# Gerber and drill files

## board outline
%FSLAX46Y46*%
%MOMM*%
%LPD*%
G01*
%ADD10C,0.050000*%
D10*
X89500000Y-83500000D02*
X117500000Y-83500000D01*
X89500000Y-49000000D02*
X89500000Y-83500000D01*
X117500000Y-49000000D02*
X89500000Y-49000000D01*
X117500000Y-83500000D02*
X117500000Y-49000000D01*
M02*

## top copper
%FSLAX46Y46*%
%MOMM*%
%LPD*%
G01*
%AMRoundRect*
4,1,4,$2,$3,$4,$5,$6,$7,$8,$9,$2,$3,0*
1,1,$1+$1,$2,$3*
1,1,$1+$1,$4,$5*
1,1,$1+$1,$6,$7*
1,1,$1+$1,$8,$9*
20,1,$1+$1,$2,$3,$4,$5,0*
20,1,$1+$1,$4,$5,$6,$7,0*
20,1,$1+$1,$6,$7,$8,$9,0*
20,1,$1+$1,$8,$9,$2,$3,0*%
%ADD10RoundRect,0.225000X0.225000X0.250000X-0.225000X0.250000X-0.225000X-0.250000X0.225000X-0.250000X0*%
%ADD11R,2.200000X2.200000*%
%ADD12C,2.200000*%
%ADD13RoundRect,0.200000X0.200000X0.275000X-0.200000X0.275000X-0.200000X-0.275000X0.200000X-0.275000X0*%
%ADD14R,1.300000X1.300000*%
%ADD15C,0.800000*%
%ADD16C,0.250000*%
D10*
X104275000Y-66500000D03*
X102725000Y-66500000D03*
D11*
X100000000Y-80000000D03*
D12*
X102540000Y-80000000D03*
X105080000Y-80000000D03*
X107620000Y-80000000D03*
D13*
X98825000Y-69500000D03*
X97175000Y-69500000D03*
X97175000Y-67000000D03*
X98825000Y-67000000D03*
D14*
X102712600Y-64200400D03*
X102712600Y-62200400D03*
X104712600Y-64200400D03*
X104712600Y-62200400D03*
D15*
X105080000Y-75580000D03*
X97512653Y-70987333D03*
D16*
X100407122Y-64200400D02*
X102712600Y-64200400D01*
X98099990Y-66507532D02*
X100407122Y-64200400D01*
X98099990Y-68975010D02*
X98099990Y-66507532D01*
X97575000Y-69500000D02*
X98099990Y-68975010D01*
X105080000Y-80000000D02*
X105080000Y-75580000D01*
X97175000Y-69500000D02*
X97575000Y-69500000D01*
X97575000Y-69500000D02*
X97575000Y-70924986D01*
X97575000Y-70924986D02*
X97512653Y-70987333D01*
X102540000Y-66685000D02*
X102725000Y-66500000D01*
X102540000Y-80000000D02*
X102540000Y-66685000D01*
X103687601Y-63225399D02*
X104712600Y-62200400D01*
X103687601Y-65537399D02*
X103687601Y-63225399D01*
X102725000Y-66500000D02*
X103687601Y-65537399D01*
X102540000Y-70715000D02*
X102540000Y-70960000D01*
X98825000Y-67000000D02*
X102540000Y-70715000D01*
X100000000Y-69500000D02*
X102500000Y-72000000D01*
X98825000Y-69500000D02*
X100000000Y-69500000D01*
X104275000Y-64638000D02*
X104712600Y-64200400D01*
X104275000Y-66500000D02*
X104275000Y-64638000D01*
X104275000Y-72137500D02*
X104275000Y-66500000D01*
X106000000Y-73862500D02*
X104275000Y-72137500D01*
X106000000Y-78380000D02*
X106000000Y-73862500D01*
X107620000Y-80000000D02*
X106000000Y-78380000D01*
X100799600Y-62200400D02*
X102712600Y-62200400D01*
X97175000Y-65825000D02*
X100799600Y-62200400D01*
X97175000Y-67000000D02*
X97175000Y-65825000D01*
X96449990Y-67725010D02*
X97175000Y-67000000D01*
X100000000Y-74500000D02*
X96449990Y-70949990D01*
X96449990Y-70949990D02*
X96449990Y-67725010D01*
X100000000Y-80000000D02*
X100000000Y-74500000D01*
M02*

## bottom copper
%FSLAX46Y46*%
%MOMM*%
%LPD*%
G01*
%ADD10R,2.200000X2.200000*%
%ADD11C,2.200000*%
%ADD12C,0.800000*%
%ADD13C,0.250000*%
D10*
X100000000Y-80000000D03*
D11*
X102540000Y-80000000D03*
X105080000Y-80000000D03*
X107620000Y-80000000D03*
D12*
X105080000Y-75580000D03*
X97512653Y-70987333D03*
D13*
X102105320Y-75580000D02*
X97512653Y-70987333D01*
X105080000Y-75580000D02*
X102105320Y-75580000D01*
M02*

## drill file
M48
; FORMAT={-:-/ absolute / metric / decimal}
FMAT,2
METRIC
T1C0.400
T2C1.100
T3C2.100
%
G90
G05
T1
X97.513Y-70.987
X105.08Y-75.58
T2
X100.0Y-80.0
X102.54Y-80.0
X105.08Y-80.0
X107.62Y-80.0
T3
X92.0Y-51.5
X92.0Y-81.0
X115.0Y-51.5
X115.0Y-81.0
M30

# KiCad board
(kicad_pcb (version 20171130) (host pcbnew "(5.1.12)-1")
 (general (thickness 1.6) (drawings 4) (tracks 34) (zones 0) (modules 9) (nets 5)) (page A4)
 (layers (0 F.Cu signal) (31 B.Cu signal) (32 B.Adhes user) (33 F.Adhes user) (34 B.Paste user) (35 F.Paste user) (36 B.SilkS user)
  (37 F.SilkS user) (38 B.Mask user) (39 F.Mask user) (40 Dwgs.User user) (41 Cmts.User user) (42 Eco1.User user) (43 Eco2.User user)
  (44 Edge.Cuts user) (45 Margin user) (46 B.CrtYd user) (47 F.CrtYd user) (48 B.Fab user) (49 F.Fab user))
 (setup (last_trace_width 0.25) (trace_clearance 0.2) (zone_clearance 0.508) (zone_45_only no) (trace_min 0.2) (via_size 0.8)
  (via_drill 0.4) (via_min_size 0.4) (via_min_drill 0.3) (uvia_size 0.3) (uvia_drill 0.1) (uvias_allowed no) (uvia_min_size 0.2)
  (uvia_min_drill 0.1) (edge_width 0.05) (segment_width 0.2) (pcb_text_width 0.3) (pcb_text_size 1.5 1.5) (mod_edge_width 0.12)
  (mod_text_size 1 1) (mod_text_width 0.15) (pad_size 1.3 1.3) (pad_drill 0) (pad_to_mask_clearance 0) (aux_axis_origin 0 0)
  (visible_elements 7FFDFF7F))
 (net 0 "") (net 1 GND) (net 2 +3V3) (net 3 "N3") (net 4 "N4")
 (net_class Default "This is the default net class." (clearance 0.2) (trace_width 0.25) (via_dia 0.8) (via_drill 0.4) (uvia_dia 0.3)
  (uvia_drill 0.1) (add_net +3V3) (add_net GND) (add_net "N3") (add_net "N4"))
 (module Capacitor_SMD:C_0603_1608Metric (layer F.Cu) (at 103.5 66.5 180)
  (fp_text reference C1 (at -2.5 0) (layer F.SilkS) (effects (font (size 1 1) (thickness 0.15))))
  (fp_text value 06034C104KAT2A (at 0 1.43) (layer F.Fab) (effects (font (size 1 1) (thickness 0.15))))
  (pad 1 smd roundrect (at -0.775 0 180) (size 0.9 0.95) (layers F.Cu F.Paste F.Mask) (roundrect_rratio 0.25) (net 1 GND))
  (pad 2 smd roundrect (at 0.775 0 180) (size 0.9 0.95) (layers F.Cu F.Paste F.Mask) (roundrect_rratio 0.25) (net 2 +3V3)))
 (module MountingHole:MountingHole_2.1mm (layer F.Cu) (at 92 81)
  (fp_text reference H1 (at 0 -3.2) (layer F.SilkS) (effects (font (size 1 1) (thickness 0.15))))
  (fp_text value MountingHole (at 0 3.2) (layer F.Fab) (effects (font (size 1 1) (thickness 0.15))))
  (pad "" np_thru_hole circle (at 0 0) (size 2.1 2.1) (drill 2.1) (layers *.Cu *.Mask)))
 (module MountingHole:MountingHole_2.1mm (layer F.Cu) (at 92 51.5)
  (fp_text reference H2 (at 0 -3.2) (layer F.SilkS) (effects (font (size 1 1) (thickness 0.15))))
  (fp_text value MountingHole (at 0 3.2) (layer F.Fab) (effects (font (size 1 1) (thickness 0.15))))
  (pad "" np_thru_hole circle (at 0 0) (size 2.1 2.1) (drill 2.1) (layers *.Cu *.Mask)))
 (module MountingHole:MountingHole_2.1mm (layer F.Cu) (at 115 51.5)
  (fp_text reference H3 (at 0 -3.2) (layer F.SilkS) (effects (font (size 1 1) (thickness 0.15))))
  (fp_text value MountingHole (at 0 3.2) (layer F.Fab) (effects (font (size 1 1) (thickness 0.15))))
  (pad "" np_thru_hole circle (at 0 0) (size 2.1 2.1) (drill 2.1) (layers *.Cu *.Mask)))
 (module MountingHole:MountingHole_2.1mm (layer F.Cu) (at 115 81)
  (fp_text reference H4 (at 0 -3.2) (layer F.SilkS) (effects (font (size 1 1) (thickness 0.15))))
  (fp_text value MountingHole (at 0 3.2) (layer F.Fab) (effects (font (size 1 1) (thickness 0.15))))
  (pad "" np_thru_hole circle (at 0 0) (size 2.1 2.1) (drill 2.1) (layers *.Cu *.Mask)))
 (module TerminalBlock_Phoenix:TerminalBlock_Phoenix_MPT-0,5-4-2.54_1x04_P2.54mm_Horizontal (layer F.Cu) (at 100 80)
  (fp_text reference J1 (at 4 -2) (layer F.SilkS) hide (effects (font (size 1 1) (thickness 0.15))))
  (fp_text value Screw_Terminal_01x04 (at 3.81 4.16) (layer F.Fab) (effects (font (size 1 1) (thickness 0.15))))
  (pad 1 thru_hole rect (at 0 0) (size 2.2 2.2) (drill 1.1) (layers *.Cu *.Mask) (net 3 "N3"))
  (pad 2 thru_hole circle (at 2.54 0) (size 2.2 2.2) (drill 1.1) (layers *.Cu *.Mask) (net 2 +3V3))
  (pad 3 thru_hole circle (at 5.08 0) (size 2.2 2.2) (drill 1.1) (layers *.Cu *.Mask) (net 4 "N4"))
  (pad 4 thru_hole circle (at 7.62 0) (size 2.2 2.2) (drill 1.1) (layers *.Cu *.Mask) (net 1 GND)))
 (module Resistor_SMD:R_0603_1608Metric (layer F.Cu) (at 98 69.5 180)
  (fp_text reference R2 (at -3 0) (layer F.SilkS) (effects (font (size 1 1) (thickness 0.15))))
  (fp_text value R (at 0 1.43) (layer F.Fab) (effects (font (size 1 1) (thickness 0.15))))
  (pad 1 smd roundrect (at -0.825 0 180) (size 0.8 0.95) (layers F.Cu F.Paste F.Mask) (roundrect_rratio 0.25) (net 2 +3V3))
  (pad 2 smd roundrect (at 0.825 0 180) (size 0.8 0.95) (layers F.Cu F.Paste F.Mask) (roundrect_rratio 0.25) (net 4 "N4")))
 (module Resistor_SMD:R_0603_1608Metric (layer F.Cu) (at 98 67 180)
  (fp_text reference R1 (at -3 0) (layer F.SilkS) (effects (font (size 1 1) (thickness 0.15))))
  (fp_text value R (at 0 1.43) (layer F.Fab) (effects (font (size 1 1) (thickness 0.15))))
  (pad 2 smd roundrect (at 0.825 0 180) (size 0.8 0.95) (layers F.Cu F.Paste F.Mask) (roundrect_rratio 0.25) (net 3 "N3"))
  (pad 1 smd roundrect (at -0.825 0 180) (size 0.8 0.95) (layers F.Cu F.Paste F.Mask) (roundrect_rratio 0.25) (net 2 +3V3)))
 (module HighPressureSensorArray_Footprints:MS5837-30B (layer F.Cu) (at 103.5 59)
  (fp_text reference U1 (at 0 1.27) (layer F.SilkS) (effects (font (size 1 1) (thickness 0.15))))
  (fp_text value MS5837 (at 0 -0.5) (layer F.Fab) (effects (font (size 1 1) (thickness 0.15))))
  (pad 4 smd rect (at -0.7874 5.2004) (size 1.3 1.3) (layers F.Cu F.Paste F.Mask) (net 4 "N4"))
  (pad 3 smd rect (at -0.7874 3.2004) (size 1.3 1.3) (layers F.Cu F.Paste F.Mask) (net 3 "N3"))
  (pad 1 smd rect (at 1.2126 5.2004) (size 1.3 1.3) (layers F.Cu F.Paste F.Mask) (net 1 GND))
  (pad 2 smd rect (at 1.2126 3.2004) (size 1.3 1.3) (layers F.Cu F.Paste F.Mask) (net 2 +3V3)))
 (gr_line (start 89.5 83.5) (end 117.5 83.5) (layer Edge.Cuts) (width 0.05))
 (gr_line (start 89.5 49) (end 89.5 83.5) (layer Edge.Cuts) (width 0.05))
 (gr_line (start 117.5 49) (end 89.5 49) (layer Edge.Cuts) (width 0.05))
 (gr_line (start 117.5 83.5) (end 117.5 49) (layer Edge.Cuts) (width 0.05))
 (segment (start 100.407122 64.2004) (end 102.7126 64.2004) (width 0.25) (layer F.Cu) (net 4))
 (segment (start 98.09999 66.507532) (end 100.407122 64.2004) (width 0.25) (layer F.Cu) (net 4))
 (segment (start 98.09999 68.97501) (end 98.09999 66.507532) (width 0.25) (layer F.Cu) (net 4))
 (segment (start 97.575 69.5) (end 98.09999 68.97501) (width 0.25) (layer F.Cu) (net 4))
 (segment (start 105.08 80) (end 105.08 75.58) (width 0.25) (layer F.Cu) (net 4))
 (via (at 105.08 75.58) (size 0.8) (drill 0.4) (layers F.Cu B.Cu) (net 4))
 (segment (start 97.175 69.5) (end 97.575 69.5) (width 0.25) (layer F.Cu) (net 4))
 (via (at 97.512653 70.987333) (size 0.8) (drill 0.4) (layers F.Cu B.Cu) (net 4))
 (segment (start 102.10532 75.58) (end 97.512653 70.987333) (width 0.25) (layer B.Cu) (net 4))
 (segment (start 97.575 69.5) (end 97.575 70.924986) (width 0.25) (layer F.Cu) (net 4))
 (segment (start 97.575 70.924986) (end 97.512653 70.987333) (width 0.25) (layer F.Cu) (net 4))
 (segment (start 105.08 75.58) (end 102.10532 75.58) (width 0.25) (layer B.Cu) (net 4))
 (segment (start 102.54 66.685) (end 102.725 66.5) (width 0.25) (layer F.Cu) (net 2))
 (segment (start 102.54 80) (end 102.54 66.685) (width 0.25) (layer F.Cu) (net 2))
 (segment (start 103.687601 63.225399) (end 104.7126 62.2004) (width 0.25) (layer F.Cu) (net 2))
 (segment (start 103.687601 65.537399) (end 103.687601 63.225399) (width 0.25) (layer F.Cu) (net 2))
 (segment (start 102.725 66.5) (end 103.687601 65.537399) (width 0.25) (layer F.Cu) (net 2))
 (segment (start 102.54 70.715) (end 102.54 70.96) (width 0.25) (layer F.Cu) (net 2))
 (segment (start 98.825 67) (end 102.54 70.715) (width 0.25) (layer F.Cu) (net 2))
 (segment (start 100 69.5) (end 102.5 72) (width 0.25) (layer F.Cu) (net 2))
 (segment (start 98.825 69.5) (end 100 69.5) (width 0.25) (layer F.Cu) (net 2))
 (segment (start 104.275 64.638) (end 104.7126 64.2004) (width 0.25) (layer F.Cu) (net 1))
 (segment (start 104.275 66.5) (end 104.275 64.638) (width 0.25) (layer F.Cu) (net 1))
 (segment (start 104.275 72.1375) (end 104.275 66.5) (width 0.25) (layer F.Cu) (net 1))
 (segment (start 106 73.8625) (end 104.275 72.1375) (width 0.25) (layer F.Cu) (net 1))
 (segment (start 106 78.38) (end 106 73.8625) (width 0.25) (layer F.Cu) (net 1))
 (segment (start 107.62 80) (end 106 78.38) (width 0.25) (layer F.Cu) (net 1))
 (segment (start 100.7996 62.2004) (end 102.7126 62.2004) (width 0.25) (layer F.Cu) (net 3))
 (segment (start 97.175 65.825) (end 100.7996 62.2004) (width 0.25) (layer F.Cu) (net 3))
 (segment (start 97.175 67) (end 97.175 65.825) (width 0.25) (layer F.Cu) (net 3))
 (segment (start 96.44999 67.72501) (end 97.175 67) (width 0.25) (layer F.Cu) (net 3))
 (segment (start 100 74.5) (end 96.44999 70.94999) (width 0.25) (layer F.Cu) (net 3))
 (segment (start 96.44999 70.94999) (end 96.44999 67.72501) (width 0.25) (layer F.Cu) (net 3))
 (segment (start 100 80) (end 100 74.5) (width 0.25) (layer F.Cu) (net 3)))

